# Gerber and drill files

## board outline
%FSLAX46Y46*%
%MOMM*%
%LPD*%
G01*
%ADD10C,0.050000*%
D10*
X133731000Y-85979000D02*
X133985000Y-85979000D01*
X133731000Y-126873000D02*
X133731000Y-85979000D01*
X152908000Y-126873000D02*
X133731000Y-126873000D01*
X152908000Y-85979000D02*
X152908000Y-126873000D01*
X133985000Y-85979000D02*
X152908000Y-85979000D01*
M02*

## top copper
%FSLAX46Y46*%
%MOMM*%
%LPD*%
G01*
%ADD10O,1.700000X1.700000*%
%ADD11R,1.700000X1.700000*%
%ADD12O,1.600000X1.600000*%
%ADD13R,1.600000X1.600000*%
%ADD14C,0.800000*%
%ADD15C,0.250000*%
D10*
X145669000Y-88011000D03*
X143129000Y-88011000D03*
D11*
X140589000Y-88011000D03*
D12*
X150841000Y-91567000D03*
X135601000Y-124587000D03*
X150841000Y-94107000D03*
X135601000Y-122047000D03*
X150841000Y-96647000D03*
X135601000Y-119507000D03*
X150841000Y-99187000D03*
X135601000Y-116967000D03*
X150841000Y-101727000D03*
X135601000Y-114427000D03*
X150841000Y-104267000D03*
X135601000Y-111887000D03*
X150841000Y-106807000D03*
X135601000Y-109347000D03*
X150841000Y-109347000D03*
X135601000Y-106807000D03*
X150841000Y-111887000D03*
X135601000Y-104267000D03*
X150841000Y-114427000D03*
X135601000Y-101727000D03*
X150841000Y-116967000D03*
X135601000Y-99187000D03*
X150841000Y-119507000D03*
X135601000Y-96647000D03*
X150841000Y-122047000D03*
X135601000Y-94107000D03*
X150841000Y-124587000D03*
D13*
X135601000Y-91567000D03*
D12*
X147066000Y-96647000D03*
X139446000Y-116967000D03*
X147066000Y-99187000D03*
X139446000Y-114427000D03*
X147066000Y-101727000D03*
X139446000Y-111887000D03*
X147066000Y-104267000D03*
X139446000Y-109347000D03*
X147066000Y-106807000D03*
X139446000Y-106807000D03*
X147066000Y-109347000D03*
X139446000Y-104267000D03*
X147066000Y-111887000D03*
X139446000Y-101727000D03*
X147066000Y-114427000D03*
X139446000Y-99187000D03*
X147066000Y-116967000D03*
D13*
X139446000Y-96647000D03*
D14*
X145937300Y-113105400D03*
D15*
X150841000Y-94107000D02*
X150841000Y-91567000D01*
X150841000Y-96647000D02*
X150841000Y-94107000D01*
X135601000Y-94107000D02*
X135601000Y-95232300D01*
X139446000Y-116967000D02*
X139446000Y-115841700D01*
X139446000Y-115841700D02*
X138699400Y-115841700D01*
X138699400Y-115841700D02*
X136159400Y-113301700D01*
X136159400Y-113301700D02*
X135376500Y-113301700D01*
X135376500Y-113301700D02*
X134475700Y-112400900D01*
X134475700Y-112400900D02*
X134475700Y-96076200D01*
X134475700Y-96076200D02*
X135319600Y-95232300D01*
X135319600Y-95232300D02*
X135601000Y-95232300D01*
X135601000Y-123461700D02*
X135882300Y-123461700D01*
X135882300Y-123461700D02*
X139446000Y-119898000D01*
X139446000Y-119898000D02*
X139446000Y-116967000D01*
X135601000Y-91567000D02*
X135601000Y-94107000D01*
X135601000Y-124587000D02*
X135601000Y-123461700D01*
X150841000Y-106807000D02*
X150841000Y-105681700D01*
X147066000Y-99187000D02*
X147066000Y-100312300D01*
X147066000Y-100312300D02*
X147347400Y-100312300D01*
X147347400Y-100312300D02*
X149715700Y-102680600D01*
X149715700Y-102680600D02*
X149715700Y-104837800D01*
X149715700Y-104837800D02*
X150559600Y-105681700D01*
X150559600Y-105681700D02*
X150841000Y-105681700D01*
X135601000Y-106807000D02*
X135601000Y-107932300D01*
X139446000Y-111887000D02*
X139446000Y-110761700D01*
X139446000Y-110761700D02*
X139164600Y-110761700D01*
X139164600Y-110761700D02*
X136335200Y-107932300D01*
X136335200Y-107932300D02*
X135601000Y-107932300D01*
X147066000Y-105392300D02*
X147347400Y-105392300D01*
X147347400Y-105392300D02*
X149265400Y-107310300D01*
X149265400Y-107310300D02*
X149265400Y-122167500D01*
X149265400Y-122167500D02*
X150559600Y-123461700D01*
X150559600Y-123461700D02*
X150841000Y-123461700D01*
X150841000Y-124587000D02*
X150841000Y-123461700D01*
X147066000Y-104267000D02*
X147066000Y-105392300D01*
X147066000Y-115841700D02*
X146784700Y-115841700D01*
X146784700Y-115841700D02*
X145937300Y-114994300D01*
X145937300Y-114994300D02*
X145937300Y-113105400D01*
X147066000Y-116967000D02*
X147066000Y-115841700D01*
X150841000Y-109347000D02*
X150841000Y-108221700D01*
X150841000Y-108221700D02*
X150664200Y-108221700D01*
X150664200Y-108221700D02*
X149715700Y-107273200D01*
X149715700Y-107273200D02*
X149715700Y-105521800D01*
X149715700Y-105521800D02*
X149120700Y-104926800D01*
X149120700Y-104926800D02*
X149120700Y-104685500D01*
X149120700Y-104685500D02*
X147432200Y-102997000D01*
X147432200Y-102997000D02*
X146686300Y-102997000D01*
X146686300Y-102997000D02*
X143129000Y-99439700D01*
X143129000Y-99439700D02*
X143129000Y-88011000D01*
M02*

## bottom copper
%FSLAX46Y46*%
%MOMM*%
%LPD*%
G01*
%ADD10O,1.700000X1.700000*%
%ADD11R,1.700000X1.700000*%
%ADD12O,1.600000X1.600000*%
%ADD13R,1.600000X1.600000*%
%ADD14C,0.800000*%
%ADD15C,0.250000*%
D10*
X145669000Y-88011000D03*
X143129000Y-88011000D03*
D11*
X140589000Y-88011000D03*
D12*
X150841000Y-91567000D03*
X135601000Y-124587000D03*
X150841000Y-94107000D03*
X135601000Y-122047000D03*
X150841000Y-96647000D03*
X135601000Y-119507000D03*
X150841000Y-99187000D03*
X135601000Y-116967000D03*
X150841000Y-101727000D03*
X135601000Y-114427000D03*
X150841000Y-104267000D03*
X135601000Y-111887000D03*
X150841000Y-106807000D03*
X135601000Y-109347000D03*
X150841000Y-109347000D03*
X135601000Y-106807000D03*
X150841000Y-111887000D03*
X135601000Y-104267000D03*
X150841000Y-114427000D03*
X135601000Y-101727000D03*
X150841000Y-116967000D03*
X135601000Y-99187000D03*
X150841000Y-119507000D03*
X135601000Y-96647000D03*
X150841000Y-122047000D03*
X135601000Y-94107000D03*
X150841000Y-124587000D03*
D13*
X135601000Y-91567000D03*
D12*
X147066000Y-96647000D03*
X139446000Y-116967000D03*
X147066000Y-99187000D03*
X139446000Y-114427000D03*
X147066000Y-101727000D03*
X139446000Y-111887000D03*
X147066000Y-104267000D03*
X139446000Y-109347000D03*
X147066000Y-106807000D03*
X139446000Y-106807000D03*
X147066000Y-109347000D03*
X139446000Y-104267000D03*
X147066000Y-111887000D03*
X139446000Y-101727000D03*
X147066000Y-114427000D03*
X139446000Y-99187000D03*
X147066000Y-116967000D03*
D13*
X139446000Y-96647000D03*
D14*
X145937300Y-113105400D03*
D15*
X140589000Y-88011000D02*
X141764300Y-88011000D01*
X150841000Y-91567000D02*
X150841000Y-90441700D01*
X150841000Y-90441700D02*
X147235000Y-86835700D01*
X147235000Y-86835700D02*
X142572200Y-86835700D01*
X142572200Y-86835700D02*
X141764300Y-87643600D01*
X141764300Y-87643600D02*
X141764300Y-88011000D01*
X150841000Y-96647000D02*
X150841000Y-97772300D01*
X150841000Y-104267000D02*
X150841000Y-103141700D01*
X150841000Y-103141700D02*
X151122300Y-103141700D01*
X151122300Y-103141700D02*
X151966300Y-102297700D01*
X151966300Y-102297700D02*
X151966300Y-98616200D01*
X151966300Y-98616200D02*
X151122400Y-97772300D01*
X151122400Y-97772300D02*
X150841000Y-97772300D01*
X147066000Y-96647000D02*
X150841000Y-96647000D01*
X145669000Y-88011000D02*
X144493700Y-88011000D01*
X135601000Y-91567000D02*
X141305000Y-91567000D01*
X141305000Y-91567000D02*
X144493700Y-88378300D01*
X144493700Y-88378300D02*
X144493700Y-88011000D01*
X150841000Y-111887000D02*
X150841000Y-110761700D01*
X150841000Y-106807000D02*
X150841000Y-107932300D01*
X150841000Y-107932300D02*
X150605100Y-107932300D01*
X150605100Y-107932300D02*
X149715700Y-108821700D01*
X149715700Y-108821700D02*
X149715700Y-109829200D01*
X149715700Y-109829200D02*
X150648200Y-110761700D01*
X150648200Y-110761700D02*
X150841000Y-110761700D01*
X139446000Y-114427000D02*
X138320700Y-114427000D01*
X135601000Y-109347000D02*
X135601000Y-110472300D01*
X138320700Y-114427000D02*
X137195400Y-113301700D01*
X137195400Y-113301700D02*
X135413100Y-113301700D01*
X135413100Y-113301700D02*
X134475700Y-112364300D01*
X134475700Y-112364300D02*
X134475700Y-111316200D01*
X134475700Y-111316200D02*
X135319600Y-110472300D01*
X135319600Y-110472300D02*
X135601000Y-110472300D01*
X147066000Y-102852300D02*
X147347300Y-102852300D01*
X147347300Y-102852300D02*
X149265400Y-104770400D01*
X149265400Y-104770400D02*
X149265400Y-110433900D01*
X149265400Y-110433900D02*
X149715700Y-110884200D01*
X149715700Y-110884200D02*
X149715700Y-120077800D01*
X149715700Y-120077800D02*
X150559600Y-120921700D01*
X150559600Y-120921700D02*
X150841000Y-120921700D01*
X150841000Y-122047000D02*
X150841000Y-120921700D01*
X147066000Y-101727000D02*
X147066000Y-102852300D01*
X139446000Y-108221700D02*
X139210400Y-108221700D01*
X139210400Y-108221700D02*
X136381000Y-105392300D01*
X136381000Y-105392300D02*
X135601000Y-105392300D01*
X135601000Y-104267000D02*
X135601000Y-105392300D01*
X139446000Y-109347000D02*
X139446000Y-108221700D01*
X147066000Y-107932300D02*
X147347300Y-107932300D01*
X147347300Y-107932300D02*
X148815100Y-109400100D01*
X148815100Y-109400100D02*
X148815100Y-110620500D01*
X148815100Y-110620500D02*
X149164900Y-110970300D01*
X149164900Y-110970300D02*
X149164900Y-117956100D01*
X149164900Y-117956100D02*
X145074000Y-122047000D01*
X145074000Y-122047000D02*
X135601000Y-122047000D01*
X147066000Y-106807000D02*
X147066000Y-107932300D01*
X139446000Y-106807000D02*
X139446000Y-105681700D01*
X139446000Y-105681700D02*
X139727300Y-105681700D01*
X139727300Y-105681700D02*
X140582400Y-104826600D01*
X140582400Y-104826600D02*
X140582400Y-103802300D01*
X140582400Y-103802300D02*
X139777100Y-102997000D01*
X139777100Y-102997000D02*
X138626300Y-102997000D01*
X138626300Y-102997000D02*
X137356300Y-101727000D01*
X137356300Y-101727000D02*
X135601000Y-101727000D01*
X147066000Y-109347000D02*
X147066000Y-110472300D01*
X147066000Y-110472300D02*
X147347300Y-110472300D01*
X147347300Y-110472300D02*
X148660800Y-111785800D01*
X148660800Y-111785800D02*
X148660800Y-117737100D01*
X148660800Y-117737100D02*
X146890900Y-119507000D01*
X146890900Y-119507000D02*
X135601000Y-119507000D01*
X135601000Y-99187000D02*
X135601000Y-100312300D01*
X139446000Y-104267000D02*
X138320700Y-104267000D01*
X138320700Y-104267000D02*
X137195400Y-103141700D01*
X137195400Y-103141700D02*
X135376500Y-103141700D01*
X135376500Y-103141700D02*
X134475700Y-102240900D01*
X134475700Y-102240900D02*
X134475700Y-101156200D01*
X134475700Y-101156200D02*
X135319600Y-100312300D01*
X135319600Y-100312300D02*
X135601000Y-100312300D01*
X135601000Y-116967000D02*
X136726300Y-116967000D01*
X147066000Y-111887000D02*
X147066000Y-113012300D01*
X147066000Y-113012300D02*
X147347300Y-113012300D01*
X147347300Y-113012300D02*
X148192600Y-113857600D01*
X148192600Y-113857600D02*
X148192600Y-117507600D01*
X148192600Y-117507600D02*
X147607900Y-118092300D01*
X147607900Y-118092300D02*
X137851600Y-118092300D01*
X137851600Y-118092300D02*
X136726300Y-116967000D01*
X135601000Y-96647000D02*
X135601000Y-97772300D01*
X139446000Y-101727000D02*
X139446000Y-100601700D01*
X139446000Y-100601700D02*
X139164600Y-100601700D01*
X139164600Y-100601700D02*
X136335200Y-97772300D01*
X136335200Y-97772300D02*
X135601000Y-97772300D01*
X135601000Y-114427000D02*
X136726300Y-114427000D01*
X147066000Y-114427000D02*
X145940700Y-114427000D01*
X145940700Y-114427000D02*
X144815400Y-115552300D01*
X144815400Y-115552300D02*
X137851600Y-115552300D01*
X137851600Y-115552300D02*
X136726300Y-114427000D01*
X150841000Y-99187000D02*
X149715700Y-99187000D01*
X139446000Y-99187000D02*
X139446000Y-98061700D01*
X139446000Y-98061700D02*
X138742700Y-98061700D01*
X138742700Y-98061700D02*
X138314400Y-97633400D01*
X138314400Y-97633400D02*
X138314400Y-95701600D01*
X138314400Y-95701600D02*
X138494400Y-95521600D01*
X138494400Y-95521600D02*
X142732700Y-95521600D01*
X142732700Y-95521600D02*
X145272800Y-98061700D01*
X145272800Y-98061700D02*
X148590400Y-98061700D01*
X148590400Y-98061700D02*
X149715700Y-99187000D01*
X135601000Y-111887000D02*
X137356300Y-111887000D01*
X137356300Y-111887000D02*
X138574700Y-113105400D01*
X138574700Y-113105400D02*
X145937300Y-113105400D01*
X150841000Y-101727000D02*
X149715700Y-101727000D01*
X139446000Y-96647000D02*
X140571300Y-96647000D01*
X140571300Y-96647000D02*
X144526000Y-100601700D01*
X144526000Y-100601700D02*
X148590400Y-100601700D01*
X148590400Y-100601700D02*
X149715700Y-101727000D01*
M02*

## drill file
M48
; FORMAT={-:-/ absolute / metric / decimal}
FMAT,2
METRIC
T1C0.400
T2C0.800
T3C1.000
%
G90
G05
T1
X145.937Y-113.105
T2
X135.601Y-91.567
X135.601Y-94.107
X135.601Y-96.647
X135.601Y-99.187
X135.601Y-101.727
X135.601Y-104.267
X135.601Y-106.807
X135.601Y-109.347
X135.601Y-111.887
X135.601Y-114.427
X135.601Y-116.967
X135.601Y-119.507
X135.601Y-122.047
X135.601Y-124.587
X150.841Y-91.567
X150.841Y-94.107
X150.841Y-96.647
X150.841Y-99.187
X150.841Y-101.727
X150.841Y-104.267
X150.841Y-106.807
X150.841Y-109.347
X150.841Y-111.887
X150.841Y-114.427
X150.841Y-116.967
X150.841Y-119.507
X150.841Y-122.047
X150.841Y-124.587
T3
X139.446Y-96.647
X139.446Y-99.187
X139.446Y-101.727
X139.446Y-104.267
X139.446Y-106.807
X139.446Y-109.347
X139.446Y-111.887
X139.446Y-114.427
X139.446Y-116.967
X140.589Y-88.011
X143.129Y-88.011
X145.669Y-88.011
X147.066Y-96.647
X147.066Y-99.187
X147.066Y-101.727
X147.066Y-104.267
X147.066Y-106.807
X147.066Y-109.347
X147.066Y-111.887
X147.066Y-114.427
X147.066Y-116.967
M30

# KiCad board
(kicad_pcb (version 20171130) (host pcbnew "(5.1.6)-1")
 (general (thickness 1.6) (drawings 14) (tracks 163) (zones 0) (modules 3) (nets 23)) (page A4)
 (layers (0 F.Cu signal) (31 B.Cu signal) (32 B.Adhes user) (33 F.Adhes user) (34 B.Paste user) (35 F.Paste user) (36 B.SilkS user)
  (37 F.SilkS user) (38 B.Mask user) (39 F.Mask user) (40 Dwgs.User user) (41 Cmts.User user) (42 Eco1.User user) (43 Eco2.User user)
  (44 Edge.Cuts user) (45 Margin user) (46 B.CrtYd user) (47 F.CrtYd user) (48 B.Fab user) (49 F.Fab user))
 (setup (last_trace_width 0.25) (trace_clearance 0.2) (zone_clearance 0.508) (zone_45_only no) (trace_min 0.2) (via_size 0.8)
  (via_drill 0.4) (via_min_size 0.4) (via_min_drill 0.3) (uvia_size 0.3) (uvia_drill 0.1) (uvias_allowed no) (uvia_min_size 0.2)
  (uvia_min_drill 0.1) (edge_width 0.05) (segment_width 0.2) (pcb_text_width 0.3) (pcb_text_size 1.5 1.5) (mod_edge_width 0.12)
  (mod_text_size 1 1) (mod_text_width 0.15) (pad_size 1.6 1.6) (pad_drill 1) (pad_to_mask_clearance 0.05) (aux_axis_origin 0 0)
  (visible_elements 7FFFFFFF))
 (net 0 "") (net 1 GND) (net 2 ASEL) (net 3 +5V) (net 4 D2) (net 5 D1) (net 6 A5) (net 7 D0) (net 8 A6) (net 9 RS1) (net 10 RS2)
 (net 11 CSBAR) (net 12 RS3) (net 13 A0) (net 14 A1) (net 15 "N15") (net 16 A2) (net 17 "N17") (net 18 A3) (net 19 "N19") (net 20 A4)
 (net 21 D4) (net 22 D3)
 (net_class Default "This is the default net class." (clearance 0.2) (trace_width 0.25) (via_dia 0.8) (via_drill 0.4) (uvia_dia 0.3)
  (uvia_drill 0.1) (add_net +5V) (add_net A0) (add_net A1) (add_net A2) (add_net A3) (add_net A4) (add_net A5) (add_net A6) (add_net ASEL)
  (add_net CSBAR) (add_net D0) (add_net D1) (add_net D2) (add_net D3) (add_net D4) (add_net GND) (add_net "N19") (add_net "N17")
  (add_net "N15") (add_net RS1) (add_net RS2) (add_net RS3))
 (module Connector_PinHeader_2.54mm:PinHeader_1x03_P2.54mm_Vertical (layer F.Cu) (at 140.589 88.011 90)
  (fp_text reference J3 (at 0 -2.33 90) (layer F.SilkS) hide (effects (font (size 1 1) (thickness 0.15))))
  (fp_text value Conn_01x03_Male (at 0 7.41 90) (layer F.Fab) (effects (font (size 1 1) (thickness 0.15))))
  (pad 3 thru_hole oval (at 0 5.08 90) (size 1.7 1.7) (drill 1) (layers *.Cu *.Mask) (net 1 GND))
  (pad 2 thru_hole oval (at 0 2.54 90) (size 1.7 1.7) (drill 1) (layers *.Cu *.Mask) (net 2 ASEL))
  (pad 1 thru_hole rect (at 0 0 90) (size 1.7 1.7) (drill 1) (layers *.Cu *.Mask) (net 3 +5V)))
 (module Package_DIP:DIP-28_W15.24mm (layer F.Cu) (at 135.601 91.567)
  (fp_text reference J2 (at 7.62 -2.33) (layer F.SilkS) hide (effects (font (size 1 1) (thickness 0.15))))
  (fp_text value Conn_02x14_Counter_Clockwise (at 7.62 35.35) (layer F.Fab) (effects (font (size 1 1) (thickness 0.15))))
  (pad 28 thru_hole oval (at 15.24 0) (size 1.6 1.6) (drill 0.8) (layers *.Cu *.Mask) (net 3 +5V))
  (pad 14 thru_hole oval (at 0 33.02) (size 1.6 1.6) (drill 0.8) (layers *.Cu *.Mask) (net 1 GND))
  (pad 27 thru_hole oval (at 15.24 2.54) (size 1.6 1.6) (drill 0.8) (layers *.Cu *.Mask) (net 3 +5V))
  (pad 13 thru_hole oval (at 0 30.48) (size 1.6 1.6) (drill 0.8) (layers *.Cu *.Mask) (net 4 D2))
  (pad 26 thru_hole oval (at 15.24 5.08) (size 1.6 1.6) (drill 0.8) (layers *.Cu *.Mask) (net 3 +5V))
  (pad 12 thru_hole oval (at 0 27.94) (size 1.6 1.6) (drill 0.8) (layers *.Cu *.Mask) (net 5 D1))
  (pad 25 thru_hole oval (at 15.24 7.62) (size 1.6 1.6) (drill 0.8) (layers *.Cu *.Mask) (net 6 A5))
  (pad 11 thru_hole oval (at 0 25.4) (size 1.6 1.6) (drill 0.8) (layers *.Cu *.Mask) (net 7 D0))
  (pad 24 thru_hole oval (at 15.24 10.16) (size 1.6 1.6) (drill 0.8) (layers *.Cu *.Mask) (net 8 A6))
  (pad 10 thru_hole oval (at 0 22.86) (size 1.6 1.6) (drill 0.8) (layers *.Cu *.Mask) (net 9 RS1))
  (pad 23 thru_hole oval (at 15.24 12.7) (size 1.6 1.6) (drill 0.8) (layers *.Cu *.Mask) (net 3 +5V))
  (pad 9 thru_hole oval (at 0 20.32) (size 1.6 1.6) (drill 0.8) (layers *.Cu *.Mask) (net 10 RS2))
  (pad 22 thru_hole oval (at 15.24 15.24) (size 1.6 1.6) (drill 0.8) (layers *.Cu *.Mask) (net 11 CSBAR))
  (pad 8 thru_hole oval (at 0 17.78) (size 1.6 1.6) (drill 0.8) (layers *.Cu *.Mask) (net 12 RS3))
  (pad 21 thru_hole oval (at 15.24 17.78) (size 1.6 1.6) (drill 0.8) (layers *.Cu *.Mask) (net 2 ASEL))
  (pad 7 thru_hole oval (at 0 15.24) (size 1.6 1.6) (drill 0.8) (layers *.Cu *.Mask) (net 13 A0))
  (pad 20 thru_hole oval (at 15.24 20.32) (size 1.6 1.6) (drill 0.8) (layers *.Cu *.Mask) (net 11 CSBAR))
  (pad 6 thru_hole oval (at 0 12.7) (size 1.6 1.6) (drill 0.8) (layers *.Cu *.Mask) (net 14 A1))
  (pad 19 thru_hole oval (at 15.24 22.86) (size 1.6 1.6) (drill 0.8) (layers *.Cu *.Mask) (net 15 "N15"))
  (pad 5 thru_hole oval (at 0 10.16) (size 1.6 1.6) (drill 0.8) (layers *.Cu *.Mask) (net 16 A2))
  (pad 18 thru_hole oval (at 15.24 25.4) (size 1.6 1.6) (drill 0.8) (layers *.Cu *.Mask) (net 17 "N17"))
  (pad 4 thru_hole oval (at 0 7.62) (size 1.6 1.6) (drill 0.8) (layers *.Cu *.Mask) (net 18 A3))
  (pad 17 thru_hole oval (at 15.24 27.94) (size 1.6 1.6) (drill 0.8) (layers *.Cu *.Mask) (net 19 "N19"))
  (pad 3 thru_hole oval (at 0 5.08) (size 1.6 1.6) (drill 0.8) (layers *.Cu *.Mask) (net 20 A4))
  (pad 16 thru_hole oval (at 15.24 30.48) (size 1.6 1.6) (drill 0.8) (layers *.Cu *.Mask) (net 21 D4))
  (pad 2 thru_hole oval (at 0 2.54) (size 1.6 1.6) (drill 0.8) (layers *.Cu *.Mask) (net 1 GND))
  (pad 15 thru_hole oval (at 15.24 33.02) (size 1.6 1.6) (drill 0.8) (layers *.Cu *.Mask) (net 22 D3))
  (pad 1 thru_hole rect (at 0 0) (size 1.6 1.6) (drill 0.8) (layers *.Cu *.Mask) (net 1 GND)))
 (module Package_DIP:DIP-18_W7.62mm (layer F.Cu) (at 139.446 96.647)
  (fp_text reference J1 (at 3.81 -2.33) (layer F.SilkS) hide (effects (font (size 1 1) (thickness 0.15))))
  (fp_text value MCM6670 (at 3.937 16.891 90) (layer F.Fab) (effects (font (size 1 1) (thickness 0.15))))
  (pad 18 thru_hole oval (at 7.62 0) (size 1.6 1.6) (drill 1) (layers *.Cu *.Mask) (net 3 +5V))
  (pad 9 thru_hole oval (at 0 20.32) (size 1.6 1.6) (drill 1) (layers *.Cu *.Mask) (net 1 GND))
  (pad 17 thru_hole oval (at 7.62 2.54) (size 1.6 1.6) (drill 1) (layers *.Cu *.Mask) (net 11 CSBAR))
  (pad 8 thru_hole oval (at 0 17.78) (size 1.6 1.6) (drill 1) (layers *.Cu *.Mask) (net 12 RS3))
  (pad 16 thru_hole oval (at 7.62 5.08) (size 1.6 1.6) (drill 1) (layers *.Cu *.Mask) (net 21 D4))
  (pad 7 thru_hole oval (at 0 15.24) (size 1.6 1.6) (drill 1) (layers *.Cu *.Mask) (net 13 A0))
  (pad 15 thru_hole oval (at 7.62 7.62) (size 1.6 1.6) (drill 1) (layers *.Cu *.Mask) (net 22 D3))
  (pad 6 thru_hole oval (at 0 12.7) (size 1.6 1.6) (drill 1) (layers *.Cu *.Mask) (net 14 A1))
  (pad 14 thru_hole oval (at 7.62 10.16) (size 1.6 1.6) (drill 1) (layers *.Cu *.Mask) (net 4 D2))
  (pad 5 thru_hole oval (at 0 10.16) (size 1.6 1.6) (drill 1) (layers *.Cu *.Mask) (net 16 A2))
  (pad 13 thru_hole oval (at 7.62 12.7) (size 1.6 1.6) (drill 1) (layers *.Cu *.Mask) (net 5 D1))
  (pad 4 thru_hole oval (at 0 7.62) (size 1.6 1.6) (drill 1) (layers *.Cu *.Mask) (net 18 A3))
  (pad 12 thru_hole oval (at 7.62 15.24) (size 1.6 1.6) (drill 1) (layers *.Cu *.Mask) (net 7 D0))
  (pad 3 thru_hole oval (at 0 5.08) (size 1.6 1.6) (drill 1) (layers *.Cu *.Mask) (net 20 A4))
  (pad 11 thru_hole oval (at 7.62 17.78) (size 1.6 1.6) (drill 1) (layers *.Cu *.Mask) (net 9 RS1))
  (pad 2 thru_hole oval (at 0 2.54) (size 1.6 1.6) (drill 1) (layers *.Cu *.Mask) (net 6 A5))
  (pad 10 thru_hole oval (at 7.62 20.32) (size 1.6 1.6) (drill 1) (layers *.Cu *.Mask) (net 10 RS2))
  (pad 1 thru_hole rect (at 0 0) (size 1.6 1.6) (drill 1) (layers *.Cu *.Mask) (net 8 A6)))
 (gr_line (start 133.731 85.979) (end 133.985 85.979) (layer Edge.Cuts) (width 0.05))
 (gr_line (start 133.731 126.873) (end 133.731 85.979) (layer Edge.Cuts) (width 0.05))
 (gr_line (start 152.908 126.873) (end 133.731 126.873) (layer Edge.Cuts) (width 0.05))
 (gr_line (start 152.908 85.979) (end 152.908 126.873) (layer Edge.Cuts) (width 0.05))
 (gr_line (start 133.985 85.979) (end 152.908 85.979) (layer Edge.Cuts) (width 0.05))
 (segment (start 140.589 88.011) (end 141.7643 88.011) (width 0.25) (layer B.Cu) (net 3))
 (segment (start 150.841 91.567) (end 150.841 90.4417) (width 0.25) (layer B.Cu) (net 3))
 (segment (start 150.841 90.4417) (end 147.235 86.8357) (width 0.25) (layer B.Cu) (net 3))
 (segment (start 147.235 86.8357) (end 142.5722 86.8357) (width 0.25) (layer B.Cu) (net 3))
 (segment (start 142.5722 86.8357) (end 141.7643 87.6436) (width 0.25) (layer B.Cu) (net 3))
 (segment (start 141.7643 87.6436) (end 141.7643 88.011) (width 0.25) (layer B.Cu) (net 3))
 (segment (start 150.841 94.107) (end 150.841 91.567) (width 0.25) (layer F.Cu) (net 3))
 (segment (start 150.841 96.647) (end 150.841 94.107) (width 0.25) (layer F.Cu) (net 3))
 (segment (start 150.841 96.647) (end 150.841 97.7723) (width 0.25) (layer B.Cu) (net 3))
 (segment (start 150.841 104.267) (end 150.841 103.1417) (width 0.25) (layer B.Cu) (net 3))
 (segment (start 150.841 103.1417) (end 151.1223 103.1417) (width 0.25) (layer B.Cu) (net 3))
 (segment (start 151.1223 103.1417) (end 151.9663 102.2977) (width 0.25) (layer B.Cu) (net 3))
 (segment (start 151.9663 102.2977) (end 151.9663 98.6162) (width 0.25) (layer B.Cu) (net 3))
 (segment (start 151.9663 98.6162) (end 151.1224 97.7723) (width 0.25) (layer B.Cu) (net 3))
 (segment (start 151.1224 97.7723) (end 150.841 97.7723) (width 0.25) (layer B.Cu) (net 3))
 (segment (start 147.066 96.647) (end 150.841 96.647) (width 0.25) (layer B.Cu) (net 3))
 (segment (start 135.601 94.107) (end 135.601 95.2323) (width 0.25) (layer F.Cu) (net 1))
 (segment (start 139.446 116.967) (end 139.446 115.8417) (width 0.25) (layer F.Cu) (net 1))
 (segment (start 139.446 115.8417) (end 138.6994 115.8417) (width 0.25) (layer F.Cu) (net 1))
 (segment (start 138.6994 115.8417) (end 136.1594 113.3017) (width 0.25) (layer F.Cu) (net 1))
 (segment (start 136.1594 113.3017) (end 135.3765 113.3017) (width 0.25) (layer F.Cu) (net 1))
 (segment (start 135.3765 113.3017) (end 134.4757 112.4009) (width 0.25) (layer F.Cu) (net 1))
 (segment (start 134.4757 112.4009) (end 134.4757 96.0762) (width 0.25) (layer F.Cu) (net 1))
 (segment (start 134.4757 96.0762) (end 135.3196 95.2323) (width 0.25) (layer F.Cu) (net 1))
 (segment (start 135.3196 95.2323) (end 135.601 95.2323) (width 0.25) (layer F.Cu) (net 1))
 (segment (start 135.601 123.4617) (end 135.8823 123.4617) (width 0.25) (layer F.Cu) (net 1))
 (segment (start 135.8823 123.4617) (end 139.446 119.898) (width 0.25) (layer F.Cu) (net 1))
 (segment (start 139.446 119.898) (end 139.446 116.967) (width 0.25) (layer F.Cu) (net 1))
 (segment (start 145.669 88.011) (end 144.4937 88.011) (width 0.25) (layer B.Cu) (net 1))
 (segment (start 135.601 91.567) (end 141.305 91.567) (width 0.25) (layer B.Cu) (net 1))
 (segment (start 141.305 91.567) (end 144.4937 88.3783) (width 0.25) (layer B.Cu) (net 1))
 (segment (start 144.4937 88.3783) (end 144.4937 88.011) (width 0.25) (layer B.Cu) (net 1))
 (segment (start 135.601 91.567) (end 135.601 94.107) (width 0.25) (layer F.Cu) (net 1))
 (segment (start 135.601 124.587) (end 135.601 123.4617) (width 0.25) (layer F.Cu) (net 1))
 (segment (start 150.841 111.887) (end 150.841 110.7617) (width 0.25) (layer B.Cu) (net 11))
 (segment (start 150.841 106.807) (end 150.841 107.9323) (width 0.25) (layer B.Cu) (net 11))
 (segment (start 150.841 107.9323) (end 150.6051 107.9323) (width 0.25) (layer B.Cu) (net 11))
 (segment (start 150.6051 107.9323) (end 149.7157 108.8217) (width 0.25) (layer B.Cu) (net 11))
 (segment (start 149.7157 108.8217) (end 149.7157 109.8292) (width 0.25) (layer B.Cu) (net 11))
 (segment (start 149.7157 109.8292) (end 150.6482 110.7617) (width 0.25) (layer B.Cu) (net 11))
 (segment (start 150.6482 110.7617) (end 150.841 110.7617) (width 0.25) (layer B.Cu) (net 11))
 (segment (start 150.841 106.807) (end 150.841 105.6817) (width 0.25) (layer F.Cu) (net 11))
 (segment (start 147.066 99.187) (end 147.066 100.3123) (width 0.25) (layer F.Cu) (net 11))
 (segment (start 147.066 100.3123) (end 147.3474 100.3123) (width 0.25) (layer F.Cu) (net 11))
 (segment (start 147.3474 100.3123) (end 149.7157 102.6806) (width 0.25) (layer F.Cu) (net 11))
 (segment (start 149.7157 102.6806) (end 149.7157 104.8378) (width 0.25) (layer F.Cu) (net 11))
 (segment (start 149.7157 104.8378) (end 150.5596 105.6817) (width 0.25) (layer F.Cu) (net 11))
 (segment (start 150.5596 105.6817) (end 150.841 105.6817) (width 0.25) (layer F.Cu) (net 11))
 (segment (start 139.446 114.427) (end 138.3207 114.427) (width 0.25) (layer B.Cu) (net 12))
 (segment (start 135.601 109.347) (end 135.601 110.4723) (width 0.25) (layer B.Cu) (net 12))
 (segment (start 138.3207 114.427) (end 137.1954 113.3017) (width 0.25) (layer B.Cu) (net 12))
 (segment (start 137.1954 113.3017) (end 135.4131 113.3017) (width 0.25) (layer B.Cu) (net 12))
 (segment (start 135.4131 113.3017) (end 134.4757 112.3643) (width 0.25) (layer B.Cu) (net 12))
 (segment (start 134.4757 112.3643) (end 134.4757 111.3162) (width 0.25) (layer B.Cu) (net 12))
 (segment (start 134.4757 111.3162) (end 135.3196 110.4723) (width 0.25) (layer B.Cu) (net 12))
 (segment (start 135.3196 110.4723) (end 135.601 110.4723) (width 0.25) (layer B.Cu) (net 12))
 (segment (start 147.066 102.8523) (end 147.3473 102.8523) (width 0.25) (layer B.Cu) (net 21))
 (segment (start 147.3473 102.8523) (end 149.2654 104.7704) (width 0.25) (layer B.Cu) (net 21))
 (segment (start 149.2654 104.7704) (end 149.2654 110.4339) (width 0.25) (layer B.Cu) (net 21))
 (segment (start 149.2654 110.4339) (end 149.7157 110.8842) (width 0.25) (layer B.Cu) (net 21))
 (segment (start 149.7157 110.8842) (end 149.7157 120.0778) (width 0.25) (layer B.Cu) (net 21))
 (segment (start 149.7157 120.0778) (end 150.5596 120.9217) (width 0.25) (layer B.Cu) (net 21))
 (segment (start 150.5596 120.9217) (end 150.841 120.9217) (width 0.25) (layer B.Cu) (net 21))
 (segment (start 150.841 122.047) (end 150.841 120.9217) (width 0.25) (layer B.Cu) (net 21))
 (segment (start 147.066 101.727) (end 147.066 102.8523) (width 0.25) (layer B.Cu) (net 21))
 (segment (start 135.601 106.807) (end 135.601 107.9323) (width 0.25) (layer F.Cu) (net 13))
 (segment (start 139.446 111.887) (end 139.446 110.7617) (width 0.25) (layer F.Cu) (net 13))
 (segment (start 139.446 110.7617) (end 139.1646 110.7617) (width 0.25) (layer F.Cu) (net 13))
 (segment (start 139.1646 110.7617) (end 136.3352 107.9323) (width 0.25) (layer F.Cu) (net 13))
 (segment (start 136.3352 107.9323) (end 135.601 107.9323) (width 0.25) (layer F.Cu) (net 13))
 (segment (start 147.066 105.3923) (end 147.3474 105.3923) (width 0.25) (layer F.Cu) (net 22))
 (segment (start 147.3474 105.3923) (end 149.2654 107.3103) (width 0.25) (layer F.Cu) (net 22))
 (segment (start 149.2654 107.3103) (end 149.2654 122.1675) (width 0.25) (layer F.Cu) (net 22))
 (segment (start 149.2654 122.1675) (end 150.5596 123.4617) (width 0.25) (layer F.Cu) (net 22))
 (segment (start 150.5596 123.4617) (end 150.841 123.4617) (width 0.25) (layer F.Cu) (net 22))
 (segment (start 150.841 124.587) (end 150.841 123.4617) (width 0.25) (layer F.Cu) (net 22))
 (segment (start 147.066 104.267) (end 147.066 105.3923) (width 0.25) (layer F.Cu) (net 22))
 (segment (start 139.446 108.2217) (end 139.2104 108.2217) (width 0.25) (layer B.Cu) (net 14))
 (segment (start 139.2104 108.2217) (end 136.381 105.3923) (width 0.25) (layer B.Cu) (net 14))
 (segment (start 136.381 105.3923) (end 135.601 105.3923) (width 0.25) (layer B.Cu) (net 14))
 (segment (start 135.601 104.267) (end 135.601 105.3923) (width 0.25) (layer B.Cu) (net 14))
 (segment (start 139.446 109.347) (end 139.446 108.2217) (width 0.25) (layer B.Cu) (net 14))
 (segment (start 147.066 107.9323) (end 147.3473 107.9323) (width 0.25) (layer B.Cu) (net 4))
 (segment (start 147.3473 107.9323) (end 148.8151 109.4001) (width 0.25) (layer B.Cu) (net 4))
 (segment (start 148.8151 109.4001) (end 148.8151 110.6205) (width 0.25) (layer B.Cu) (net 4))
 (segment (start 148.8151 110.6205) (end 149.1649 110.9703) (width 0.25) (layer B.Cu) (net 4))
 (segment (start 149.1649 110.9703) (end 149.1649 117.9561) (width 0.25) (layer B.Cu) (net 4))
 (segment (start 149.1649 117.9561) (end 145.074 122.047) (width 0.25) (layer B.Cu) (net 4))
 (segment (start 145.074 122.047) (end 135.601 122.047) (width 0.25) (layer B.Cu) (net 4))
 (segment (start 147.066 106.807) (end 147.066 107.9323) (width 0.25) (layer B.Cu) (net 4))
 (segment (start 139.446 106.807) (end 139.446 105.6817) (width 0.25) (layer B.Cu) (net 16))
 (segment (start 139.446 105.6817) (end 139.7273 105.6817) (width 0.25) (layer B.Cu) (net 16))
 (segment (start 139.7273 105.6817) (end 140.5824 104.8266) (width 0.25) (layer B.Cu) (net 16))
 (segment (start 140.5824 104.8266) (end 140.5824 103.8023) (width 0.25) (layer B.Cu) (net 16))
 (segment (start 140.5824 103.8023) (end 139.7771 102.997) (width 0.25) (layer B.Cu) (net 16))
 (segment (start 139.7771 102.997) (end 138.6263 102.997) (width 0.25) (layer B.Cu) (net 16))
 (segment (start 138.6263 102.997) (end 137.3563 101.727) (width 0.25) (layer B.Cu) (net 16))
 (segment (start 137.3563 101.727) (end 135.601 101.727) (width 0.25) (layer B.Cu) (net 16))
 (segment (start 147.066 109.347) (end 147.066 110.4723) (width 0.25) (layer B.Cu) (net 5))
 (segment (start 147.066 110.4723) (end 147.3473 110.4723) (width 0.25) (layer B.Cu) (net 5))
 (segment (start 147.3473 110.4723) (end 148.6608 111.7858) (width 0.25) (layer B.Cu) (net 5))
 (segment (start 148.6608 111.7858) (end 148.6608 117.7371) (width 0.25) (layer B.Cu) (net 5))
 (segment (start 148.6608 117.7371) (end 146.8909 119.507) (width 0.25) (layer B.Cu) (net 5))
 (segment (start 146.8909 119.507) (end 135.601 119.507) (width 0.25) (layer B.Cu) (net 5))
 (segment (start 135.601 99.187) (end 135.601 100.3123) (width 0.25) (layer B.Cu) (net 18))
 (segment (start 139.446 104.267) (end 138.3207 104.267) (width 0.25) (layer B.Cu) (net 18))
 (segment (start 138.3207 104.267) (end 137.1954 103.1417) (width 0.25) (layer B.Cu) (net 18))
 (segment (start 137.1954 103.1417) (end 135.3765 103.1417) (width 0.25) (layer B.Cu) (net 18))
 (segment (start 135.3765 103.1417) (end 134.4757 102.2409) (width 0.25) (layer B.Cu) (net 18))
 (segment (start 134.4757 102.2409) (end 134.4757 101.1562) (width 0.25) (layer B.Cu) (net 18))
 (segment (start 134.4757 101.1562) (end 135.3196 100.3123) (width 0.25) (layer B.Cu) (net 18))
 (segment (start 135.3196 100.3123) (end 135.601 100.3123) (width 0.25) (layer B.Cu) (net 18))
 (segment (start 135.601 116.967) (end 136.7263 116.967) (width 0.25) (layer B.Cu) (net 7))
 (segment (start 147.066 111.887) (end 147.066 113.0123) (width 0.25) (layer B.Cu) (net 7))
 (segment (start 147.066 113.0123) (end 147.3473 113.0123) (width 0.25) (layer B.Cu) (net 7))
 (segment (start 147.3473 113.0123) (end 148.1926 113.8576) (width 0.25) (layer B.Cu) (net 7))
 (segment (start 148.1926 113.8576) (end 148.1926 117.5076) (width 0.25) (layer B.Cu) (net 7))
 (segment (start 148.1926 117.5076) (end 147.6079 118.0923) (width 0.25) (layer B.Cu) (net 7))
 (segment (start 147.6079 118.0923) (end 137.8516 118.0923) (width 0.25) (layer B.Cu) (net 7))
 (segment (start 137.8516 118.0923) (end 136.7263 116.967) (width 0.25) (layer B.Cu) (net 7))
 (segment (start 135.601 96.647) (end 135.601 97.7723) (width 0.25) (layer B.Cu) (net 20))
 (segment (start 139.446 101.727) (end 139.446 100.6017) (width 0.25) (layer B.Cu) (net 20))
 (segment (start 139.446 100.6017) (end 139.1646 100.6017) (width 0.25) (layer B.Cu) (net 20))
 (segment (start 139.1646 100.6017) (end 136.3352 97.7723) (width 0.25) (layer B.Cu) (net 20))
 (segment (start 136.3352 97.7723) (end 135.601 97.7723) (width 0.25) (layer B.Cu) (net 20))
 (segment (start 135.601 114.427) (end 136.7263 114.427) (width 0.25) (layer B.Cu) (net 9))
 (segment (start 147.066 114.427) (end 145.9407 114.427) (width 0.25) (layer B.Cu) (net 9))
 (segment (start 145.9407 114.427) (end 144.8154 115.5523) (width 0.25) (layer B.Cu) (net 9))
 (segment (start 144.8154 115.5523) (end 137.8516 115.5523) (width 0.25) (layer B.Cu) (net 9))
 (segment (start 137.8516 115.5523) (end 136.7263 114.427) (width 0.25) (layer B.Cu) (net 9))
 (segment (start 150.841 99.187) (end 149.7157 99.187) (width 0.25) (layer B.Cu) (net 6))
 (segment (start 139.446 99.187) (end 139.446 98.0617) (width 0.25) (layer B.Cu) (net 6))
 (segment (start 139.446 98.0617) (end 138.7427 98.0617) (width 0.25) (layer B.Cu) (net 6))
 (segment (start 138.7427 98.0617) (end 138.3144 97.6334) (width 0.25) (layer B.Cu) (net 6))
 (segment (start 138.3144 97.6334) (end 138.3144 95.7016) (width 0.25) (layer B.Cu) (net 6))
 (segment (start 138.3144 95.7016) (end 138.4944 95.5216) (width 0.25) (layer B.Cu) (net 6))
 (segment (start 138.4944 95.5216) (end 142.7327 95.5216) (width 0.25) (layer B.Cu) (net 6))
 (segment (start 142.7327 95.5216) (end 145.2728 98.0617) (width 0.25) (layer B.Cu) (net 6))
 (segment (start 145.2728 98.0617) (end 148.5904 98.0617) (width 0.25) (layer B.Cu) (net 6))
 (segment (start 148.5904 98.0617) (end 149.7157 99.187) (width 0.25) (layer B.Cu) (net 6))
 (segment (start 147.066 115.8417) (end 146.7847 115.8417) (width 0.25) (layer F.Cu) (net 10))
 (segment (start 146.7847 115.8417) (end 145.9373 114.9943) (width 0.25) (layer F.Cu) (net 10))
 (segment (start 145.9373 114.9943) (end 145.9373 113.1054) (width 0.25) (layer F.Cu) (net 10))
 (segment (start 135.601 111.887) (end 137.3563 111.887) (width 0.25) (layer B.Cu) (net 10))
 (segment (start 137.3563 111.887) (end 138.5747 113.1054) (width 0.25) (layer B.Cu) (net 10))
 (segment (start 138.5747 113.1054) (end 145.9373 113.1054) (width 0.25) (layer B.Cu) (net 10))
 (segment (start 147.066 116.967) (end 147.066 115.8417) (width 0.25) (layer F.Cu) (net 10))
 (via (at 145.9373 113.1054) (size 0.8) (layers F.Cu B.Cu) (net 10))
 (segment (start 150.841 101.727) (end 149.7157 101.727) (width 0.25) (layer B.Cu) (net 8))
 (segment (start 139.446 96.647) (end 140.5713 96.647) (width 0.25) (layer B.Cu) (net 8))
 (segment (start 140.5713 96.647) (end 144.526 100.6017) (width 0.25) (layer B.Cu) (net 8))
 (segment (start 144.526 100.6017) (end 148.5904 100.6017) (width 0.25) (layer B.Cu) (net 8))
 (segment (start 148.5904 100.6017) (end 149.7157 101.727) (width 0.25) (layer B.Cu) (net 8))
 (segment (start 150.841 109.347) (end 150.841 108.2217) (width 0.25) (layer F.Cu) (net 2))
 (segment (start 150.841 108.2217) (end 150.6642 108.2217) (width 0.25) (layer F.Cu) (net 2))
 (segment (start 150.6642 108.2217) (end 149.7157 107.2732) (width 0.25) (layer F.Cu) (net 2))
 (segment (start 149.7157 107.2732) (end 149.7157 105.5218) (width 0.25) (layer F.Cu) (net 2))
 (segment (start 149.7157 105.5218) (end 149.1207 104.9268) (width 0.25) (layer F.Cu) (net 2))
 (segment (start 149.1207 104.9268) (end 149.1207 104.6855) (width 0.25) (layer F.Cu) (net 2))
 (segment (start 149.1207 104.6855) (end 147.4322 102.997) (width 0.25) (layer F.Cu) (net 2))
 (segment (start 147.4322 102.997) (end 146.6863 102.997) (width 0.25) (layer F.Cu) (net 2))
 (segment (start 146.6863 102.997) (end 143.129 99.4397) (width 0.25) (layer F.Cu) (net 2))
 (segment (start 143.129 99.4397) (end 143.129 88.011) (width 0.25) (layer F.Cu) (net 2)))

